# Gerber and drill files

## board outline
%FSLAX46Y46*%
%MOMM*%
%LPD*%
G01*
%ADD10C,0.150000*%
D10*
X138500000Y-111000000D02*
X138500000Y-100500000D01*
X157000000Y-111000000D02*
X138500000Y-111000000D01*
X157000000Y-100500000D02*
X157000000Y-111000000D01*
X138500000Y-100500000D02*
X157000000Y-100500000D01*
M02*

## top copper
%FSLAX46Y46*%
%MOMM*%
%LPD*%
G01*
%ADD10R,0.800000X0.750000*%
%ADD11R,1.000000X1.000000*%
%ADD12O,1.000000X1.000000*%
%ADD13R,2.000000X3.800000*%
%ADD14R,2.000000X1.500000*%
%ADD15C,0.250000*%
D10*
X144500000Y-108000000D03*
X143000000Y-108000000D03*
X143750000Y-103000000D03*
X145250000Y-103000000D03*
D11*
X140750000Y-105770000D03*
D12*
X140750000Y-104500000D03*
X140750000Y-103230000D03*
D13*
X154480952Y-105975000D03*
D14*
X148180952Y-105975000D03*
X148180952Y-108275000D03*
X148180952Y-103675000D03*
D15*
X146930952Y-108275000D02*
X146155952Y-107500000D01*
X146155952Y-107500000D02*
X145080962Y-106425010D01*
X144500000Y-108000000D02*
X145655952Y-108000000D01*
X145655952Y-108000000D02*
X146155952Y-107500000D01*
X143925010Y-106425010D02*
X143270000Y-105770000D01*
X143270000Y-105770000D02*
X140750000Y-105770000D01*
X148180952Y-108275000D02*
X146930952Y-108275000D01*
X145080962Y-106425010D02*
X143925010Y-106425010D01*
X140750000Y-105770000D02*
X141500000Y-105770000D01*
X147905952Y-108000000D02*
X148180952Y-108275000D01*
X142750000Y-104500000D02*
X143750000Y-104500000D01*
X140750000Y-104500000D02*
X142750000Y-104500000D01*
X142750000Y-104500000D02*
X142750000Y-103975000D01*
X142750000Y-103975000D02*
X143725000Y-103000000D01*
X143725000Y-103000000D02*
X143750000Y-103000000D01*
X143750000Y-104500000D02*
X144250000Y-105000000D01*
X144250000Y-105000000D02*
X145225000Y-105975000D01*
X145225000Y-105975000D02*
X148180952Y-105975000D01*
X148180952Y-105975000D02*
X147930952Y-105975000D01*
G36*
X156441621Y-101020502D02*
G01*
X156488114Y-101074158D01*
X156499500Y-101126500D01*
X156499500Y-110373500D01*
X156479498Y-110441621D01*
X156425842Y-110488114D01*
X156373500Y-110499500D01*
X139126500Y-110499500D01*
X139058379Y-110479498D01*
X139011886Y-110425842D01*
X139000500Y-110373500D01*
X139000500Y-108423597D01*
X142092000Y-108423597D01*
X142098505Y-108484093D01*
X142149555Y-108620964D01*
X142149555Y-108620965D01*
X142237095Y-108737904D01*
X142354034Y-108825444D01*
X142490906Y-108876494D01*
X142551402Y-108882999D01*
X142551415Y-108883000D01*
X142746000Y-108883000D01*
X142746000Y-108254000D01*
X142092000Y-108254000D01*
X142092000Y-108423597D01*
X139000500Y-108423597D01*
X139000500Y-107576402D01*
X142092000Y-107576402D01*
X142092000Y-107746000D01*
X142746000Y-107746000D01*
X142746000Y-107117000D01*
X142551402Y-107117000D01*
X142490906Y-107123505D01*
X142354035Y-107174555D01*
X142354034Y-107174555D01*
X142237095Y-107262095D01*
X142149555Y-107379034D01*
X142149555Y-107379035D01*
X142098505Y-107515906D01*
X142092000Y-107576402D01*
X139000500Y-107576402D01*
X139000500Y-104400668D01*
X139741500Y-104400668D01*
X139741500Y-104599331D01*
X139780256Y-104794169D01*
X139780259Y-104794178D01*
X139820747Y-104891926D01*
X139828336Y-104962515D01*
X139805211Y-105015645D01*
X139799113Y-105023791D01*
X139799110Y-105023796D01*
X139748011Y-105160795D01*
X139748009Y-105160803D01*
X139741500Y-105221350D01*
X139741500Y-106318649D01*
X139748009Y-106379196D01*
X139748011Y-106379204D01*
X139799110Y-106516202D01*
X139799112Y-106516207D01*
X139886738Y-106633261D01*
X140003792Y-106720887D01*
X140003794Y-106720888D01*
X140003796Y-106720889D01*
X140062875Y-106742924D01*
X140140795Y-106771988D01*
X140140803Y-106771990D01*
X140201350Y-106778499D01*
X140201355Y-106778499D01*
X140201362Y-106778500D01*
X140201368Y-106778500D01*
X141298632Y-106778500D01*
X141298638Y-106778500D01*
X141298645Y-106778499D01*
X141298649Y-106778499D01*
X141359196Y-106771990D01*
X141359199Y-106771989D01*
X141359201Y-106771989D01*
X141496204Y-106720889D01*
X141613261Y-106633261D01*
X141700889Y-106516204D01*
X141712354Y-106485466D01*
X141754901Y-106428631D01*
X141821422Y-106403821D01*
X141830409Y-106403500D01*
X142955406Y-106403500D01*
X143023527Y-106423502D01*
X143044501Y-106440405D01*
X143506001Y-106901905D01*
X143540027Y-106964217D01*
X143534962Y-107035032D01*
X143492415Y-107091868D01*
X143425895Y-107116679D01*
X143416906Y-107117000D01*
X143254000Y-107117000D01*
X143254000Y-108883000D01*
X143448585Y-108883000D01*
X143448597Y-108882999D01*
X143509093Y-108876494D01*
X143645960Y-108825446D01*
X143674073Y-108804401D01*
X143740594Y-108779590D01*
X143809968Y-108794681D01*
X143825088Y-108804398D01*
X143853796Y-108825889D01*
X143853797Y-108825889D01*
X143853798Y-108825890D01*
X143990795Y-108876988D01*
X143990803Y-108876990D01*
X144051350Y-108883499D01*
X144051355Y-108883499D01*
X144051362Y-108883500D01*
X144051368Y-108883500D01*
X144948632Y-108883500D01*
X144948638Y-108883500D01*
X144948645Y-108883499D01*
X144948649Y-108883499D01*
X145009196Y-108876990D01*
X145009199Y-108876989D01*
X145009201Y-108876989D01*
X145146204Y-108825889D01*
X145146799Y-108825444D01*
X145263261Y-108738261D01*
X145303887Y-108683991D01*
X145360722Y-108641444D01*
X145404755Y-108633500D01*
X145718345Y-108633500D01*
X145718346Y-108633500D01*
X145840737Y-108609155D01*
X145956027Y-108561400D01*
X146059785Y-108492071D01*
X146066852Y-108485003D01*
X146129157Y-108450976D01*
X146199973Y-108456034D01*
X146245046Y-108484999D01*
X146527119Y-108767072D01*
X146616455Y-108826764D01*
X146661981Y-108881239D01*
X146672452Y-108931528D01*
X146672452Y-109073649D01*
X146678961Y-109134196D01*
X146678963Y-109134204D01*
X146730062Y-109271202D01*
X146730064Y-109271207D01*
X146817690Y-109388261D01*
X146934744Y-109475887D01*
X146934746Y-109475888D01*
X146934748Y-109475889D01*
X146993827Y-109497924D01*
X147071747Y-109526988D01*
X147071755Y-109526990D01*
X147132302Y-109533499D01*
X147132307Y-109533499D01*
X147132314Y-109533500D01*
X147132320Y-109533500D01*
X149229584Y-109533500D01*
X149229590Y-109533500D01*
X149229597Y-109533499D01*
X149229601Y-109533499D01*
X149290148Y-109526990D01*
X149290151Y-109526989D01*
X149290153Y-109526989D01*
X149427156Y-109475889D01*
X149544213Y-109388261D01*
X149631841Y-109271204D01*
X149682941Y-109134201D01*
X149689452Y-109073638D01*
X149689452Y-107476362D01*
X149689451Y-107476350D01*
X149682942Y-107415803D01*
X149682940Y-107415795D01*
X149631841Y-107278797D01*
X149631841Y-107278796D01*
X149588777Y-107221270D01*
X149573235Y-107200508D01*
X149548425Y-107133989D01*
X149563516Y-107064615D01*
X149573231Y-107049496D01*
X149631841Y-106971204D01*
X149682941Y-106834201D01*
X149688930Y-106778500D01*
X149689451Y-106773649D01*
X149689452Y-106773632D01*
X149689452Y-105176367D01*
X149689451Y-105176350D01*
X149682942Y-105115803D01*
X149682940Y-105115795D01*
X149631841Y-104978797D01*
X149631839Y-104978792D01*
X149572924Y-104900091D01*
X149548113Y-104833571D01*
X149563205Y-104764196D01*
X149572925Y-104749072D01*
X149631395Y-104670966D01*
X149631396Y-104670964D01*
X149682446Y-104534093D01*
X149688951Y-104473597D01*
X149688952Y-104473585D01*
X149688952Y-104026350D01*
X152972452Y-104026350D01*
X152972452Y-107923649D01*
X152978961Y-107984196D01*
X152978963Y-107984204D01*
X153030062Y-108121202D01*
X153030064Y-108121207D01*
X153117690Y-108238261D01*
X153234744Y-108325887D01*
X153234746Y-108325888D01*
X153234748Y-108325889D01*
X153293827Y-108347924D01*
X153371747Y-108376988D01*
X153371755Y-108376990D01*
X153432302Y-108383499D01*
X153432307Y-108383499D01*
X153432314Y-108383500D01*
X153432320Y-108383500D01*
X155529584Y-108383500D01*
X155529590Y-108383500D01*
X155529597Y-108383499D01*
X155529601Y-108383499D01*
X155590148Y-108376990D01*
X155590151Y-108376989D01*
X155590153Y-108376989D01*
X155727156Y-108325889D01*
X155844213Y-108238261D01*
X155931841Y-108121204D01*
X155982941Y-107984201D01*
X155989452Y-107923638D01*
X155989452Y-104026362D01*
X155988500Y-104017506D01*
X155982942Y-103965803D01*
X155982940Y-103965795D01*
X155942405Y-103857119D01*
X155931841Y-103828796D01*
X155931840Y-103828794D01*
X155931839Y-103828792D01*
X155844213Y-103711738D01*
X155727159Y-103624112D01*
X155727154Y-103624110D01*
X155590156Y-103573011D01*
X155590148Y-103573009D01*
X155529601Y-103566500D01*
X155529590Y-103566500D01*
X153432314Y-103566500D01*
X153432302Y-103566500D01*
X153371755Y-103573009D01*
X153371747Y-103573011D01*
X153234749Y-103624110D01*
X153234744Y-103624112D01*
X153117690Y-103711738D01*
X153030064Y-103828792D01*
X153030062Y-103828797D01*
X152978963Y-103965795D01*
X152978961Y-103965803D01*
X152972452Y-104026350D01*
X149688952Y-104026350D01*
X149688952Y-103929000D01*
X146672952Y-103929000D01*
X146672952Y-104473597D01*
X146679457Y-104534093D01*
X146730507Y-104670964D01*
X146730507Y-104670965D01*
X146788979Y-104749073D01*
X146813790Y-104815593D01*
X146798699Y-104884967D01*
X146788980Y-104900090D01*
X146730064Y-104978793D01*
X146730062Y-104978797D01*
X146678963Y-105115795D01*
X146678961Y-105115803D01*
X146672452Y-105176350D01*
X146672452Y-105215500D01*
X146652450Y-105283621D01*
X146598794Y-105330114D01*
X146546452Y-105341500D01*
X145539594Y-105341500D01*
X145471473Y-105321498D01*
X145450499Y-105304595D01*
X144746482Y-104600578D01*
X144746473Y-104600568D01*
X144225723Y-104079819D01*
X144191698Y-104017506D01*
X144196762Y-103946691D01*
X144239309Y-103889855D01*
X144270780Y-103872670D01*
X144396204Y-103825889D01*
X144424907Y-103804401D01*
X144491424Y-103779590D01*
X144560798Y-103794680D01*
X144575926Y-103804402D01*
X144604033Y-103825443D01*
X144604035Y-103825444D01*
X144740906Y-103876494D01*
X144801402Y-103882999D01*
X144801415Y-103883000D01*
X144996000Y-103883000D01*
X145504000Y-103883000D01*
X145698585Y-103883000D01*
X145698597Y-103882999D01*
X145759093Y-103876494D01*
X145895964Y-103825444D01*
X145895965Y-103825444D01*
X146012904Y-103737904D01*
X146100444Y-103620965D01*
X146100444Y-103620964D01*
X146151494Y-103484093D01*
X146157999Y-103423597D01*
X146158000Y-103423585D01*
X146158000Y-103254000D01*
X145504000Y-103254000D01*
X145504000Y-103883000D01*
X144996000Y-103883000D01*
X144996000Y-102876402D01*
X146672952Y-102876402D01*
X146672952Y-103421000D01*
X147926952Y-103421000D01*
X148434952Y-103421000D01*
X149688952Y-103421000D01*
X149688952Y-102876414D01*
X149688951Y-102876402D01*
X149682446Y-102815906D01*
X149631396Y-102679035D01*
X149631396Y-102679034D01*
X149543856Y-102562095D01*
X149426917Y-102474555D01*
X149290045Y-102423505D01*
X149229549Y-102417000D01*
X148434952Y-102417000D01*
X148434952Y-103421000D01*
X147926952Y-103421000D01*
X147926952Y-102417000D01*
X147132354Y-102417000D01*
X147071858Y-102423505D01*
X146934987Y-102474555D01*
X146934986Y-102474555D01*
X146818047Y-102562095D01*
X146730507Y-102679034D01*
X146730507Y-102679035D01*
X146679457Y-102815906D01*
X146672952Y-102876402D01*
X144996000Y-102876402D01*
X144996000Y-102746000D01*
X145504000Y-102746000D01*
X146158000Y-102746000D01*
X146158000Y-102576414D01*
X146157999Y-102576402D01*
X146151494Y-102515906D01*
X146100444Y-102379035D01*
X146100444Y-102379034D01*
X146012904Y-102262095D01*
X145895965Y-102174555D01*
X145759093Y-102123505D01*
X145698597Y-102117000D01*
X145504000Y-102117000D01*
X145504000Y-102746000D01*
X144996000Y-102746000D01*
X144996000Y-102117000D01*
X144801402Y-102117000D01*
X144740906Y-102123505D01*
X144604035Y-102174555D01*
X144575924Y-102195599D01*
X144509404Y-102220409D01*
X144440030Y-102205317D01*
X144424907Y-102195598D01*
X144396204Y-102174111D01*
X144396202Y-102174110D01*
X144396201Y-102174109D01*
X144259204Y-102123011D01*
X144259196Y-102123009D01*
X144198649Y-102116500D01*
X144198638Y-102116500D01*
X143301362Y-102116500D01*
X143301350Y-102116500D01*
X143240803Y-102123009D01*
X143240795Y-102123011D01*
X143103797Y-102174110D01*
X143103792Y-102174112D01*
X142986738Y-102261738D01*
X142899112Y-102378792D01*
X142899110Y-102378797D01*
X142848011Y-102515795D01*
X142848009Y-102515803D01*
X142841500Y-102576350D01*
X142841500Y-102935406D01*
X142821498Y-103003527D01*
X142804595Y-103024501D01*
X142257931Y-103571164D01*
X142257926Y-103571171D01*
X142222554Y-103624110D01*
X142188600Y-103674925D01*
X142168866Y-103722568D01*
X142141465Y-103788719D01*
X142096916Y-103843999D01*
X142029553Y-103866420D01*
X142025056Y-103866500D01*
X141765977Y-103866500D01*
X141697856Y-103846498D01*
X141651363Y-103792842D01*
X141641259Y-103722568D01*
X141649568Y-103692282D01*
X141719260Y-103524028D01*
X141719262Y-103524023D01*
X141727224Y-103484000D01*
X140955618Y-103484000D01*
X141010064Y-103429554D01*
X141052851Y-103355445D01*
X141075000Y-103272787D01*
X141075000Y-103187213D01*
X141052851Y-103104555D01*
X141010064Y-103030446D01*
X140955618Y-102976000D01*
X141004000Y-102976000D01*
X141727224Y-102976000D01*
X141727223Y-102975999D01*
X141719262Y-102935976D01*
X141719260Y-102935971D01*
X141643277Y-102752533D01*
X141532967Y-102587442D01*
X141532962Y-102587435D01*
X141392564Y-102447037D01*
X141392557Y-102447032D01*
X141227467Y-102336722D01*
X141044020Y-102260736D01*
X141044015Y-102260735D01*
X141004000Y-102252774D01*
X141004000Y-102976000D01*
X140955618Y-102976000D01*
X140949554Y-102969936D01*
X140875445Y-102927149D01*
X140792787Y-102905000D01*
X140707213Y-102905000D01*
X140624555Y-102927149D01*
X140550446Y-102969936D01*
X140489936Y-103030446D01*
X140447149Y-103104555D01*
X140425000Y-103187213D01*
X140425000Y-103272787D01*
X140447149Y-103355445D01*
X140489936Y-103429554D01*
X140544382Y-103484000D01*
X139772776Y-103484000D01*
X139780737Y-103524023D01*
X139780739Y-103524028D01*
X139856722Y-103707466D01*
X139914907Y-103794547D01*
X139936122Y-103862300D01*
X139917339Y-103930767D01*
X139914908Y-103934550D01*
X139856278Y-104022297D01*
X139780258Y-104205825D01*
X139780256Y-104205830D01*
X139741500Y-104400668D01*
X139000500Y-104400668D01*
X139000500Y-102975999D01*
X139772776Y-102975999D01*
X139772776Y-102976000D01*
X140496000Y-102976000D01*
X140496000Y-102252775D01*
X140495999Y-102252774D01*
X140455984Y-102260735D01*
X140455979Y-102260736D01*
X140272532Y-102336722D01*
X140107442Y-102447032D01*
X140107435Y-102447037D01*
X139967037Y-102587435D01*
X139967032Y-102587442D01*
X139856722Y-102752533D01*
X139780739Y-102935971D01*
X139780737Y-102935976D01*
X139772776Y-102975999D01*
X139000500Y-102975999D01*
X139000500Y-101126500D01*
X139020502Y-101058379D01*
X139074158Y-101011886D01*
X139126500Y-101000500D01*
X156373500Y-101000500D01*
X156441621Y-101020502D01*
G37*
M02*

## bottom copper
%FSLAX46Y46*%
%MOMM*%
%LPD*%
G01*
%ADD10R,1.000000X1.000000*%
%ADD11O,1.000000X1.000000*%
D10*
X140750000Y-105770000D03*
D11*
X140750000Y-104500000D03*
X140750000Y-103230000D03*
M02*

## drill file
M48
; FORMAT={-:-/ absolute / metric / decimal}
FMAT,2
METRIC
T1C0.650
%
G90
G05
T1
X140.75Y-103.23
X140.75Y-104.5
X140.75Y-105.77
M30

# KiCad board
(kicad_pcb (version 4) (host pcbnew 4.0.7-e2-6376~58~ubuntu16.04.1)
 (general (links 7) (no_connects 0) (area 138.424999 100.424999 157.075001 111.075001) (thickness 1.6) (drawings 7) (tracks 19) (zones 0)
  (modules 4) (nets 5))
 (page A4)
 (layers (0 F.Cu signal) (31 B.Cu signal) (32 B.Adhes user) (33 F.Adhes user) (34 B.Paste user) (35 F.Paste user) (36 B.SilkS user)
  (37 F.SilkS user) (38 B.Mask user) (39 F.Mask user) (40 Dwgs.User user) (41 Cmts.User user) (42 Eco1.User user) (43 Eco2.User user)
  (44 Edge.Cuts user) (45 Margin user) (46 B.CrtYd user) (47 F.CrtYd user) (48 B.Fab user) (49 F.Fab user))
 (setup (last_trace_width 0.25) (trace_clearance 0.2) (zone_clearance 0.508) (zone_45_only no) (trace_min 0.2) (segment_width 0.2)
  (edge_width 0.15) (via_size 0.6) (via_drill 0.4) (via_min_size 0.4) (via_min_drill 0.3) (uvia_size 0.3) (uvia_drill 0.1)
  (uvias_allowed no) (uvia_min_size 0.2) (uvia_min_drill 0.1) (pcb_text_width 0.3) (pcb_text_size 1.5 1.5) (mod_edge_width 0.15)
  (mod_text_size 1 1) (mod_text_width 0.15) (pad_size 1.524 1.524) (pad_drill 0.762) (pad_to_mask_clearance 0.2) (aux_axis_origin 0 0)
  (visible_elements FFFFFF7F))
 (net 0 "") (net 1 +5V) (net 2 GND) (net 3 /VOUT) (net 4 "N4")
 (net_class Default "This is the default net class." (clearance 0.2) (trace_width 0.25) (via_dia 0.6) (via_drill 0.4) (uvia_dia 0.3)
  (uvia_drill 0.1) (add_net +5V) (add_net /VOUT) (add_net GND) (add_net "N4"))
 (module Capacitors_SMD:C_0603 (layer F.Cu) (at 143.75 108 180)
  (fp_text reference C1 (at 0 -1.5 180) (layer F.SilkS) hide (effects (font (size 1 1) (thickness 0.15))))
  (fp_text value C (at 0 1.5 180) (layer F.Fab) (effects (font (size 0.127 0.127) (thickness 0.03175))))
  (pad 1 smd rect (at -0.75 0 180) (size 0.8 0.75) (layers F.Cu F.Paste F.Mask) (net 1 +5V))
  (pad 2 smd rect (at 0.75 0 180) (size 0.8 0.75) (layers F.Cu F.Paste F.Mask) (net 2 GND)))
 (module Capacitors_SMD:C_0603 (layer F.Cu) (at 144.5 103)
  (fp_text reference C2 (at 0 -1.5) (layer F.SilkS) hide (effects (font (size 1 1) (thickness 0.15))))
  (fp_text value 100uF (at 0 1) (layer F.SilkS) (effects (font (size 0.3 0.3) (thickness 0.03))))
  (pad 1 smd rect (at -0.75 0) (size 0.8 0.75) (layers F.Cu F.Paste F.Mask) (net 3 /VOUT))
  (pad 2 smd rect (at 0.75 0) (size 0.8 0.75) (layers F.Cu F.Paste F.Mask) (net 2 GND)))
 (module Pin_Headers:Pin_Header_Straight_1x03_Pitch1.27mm (layer F.Cu) (at 140.75 105.77 180)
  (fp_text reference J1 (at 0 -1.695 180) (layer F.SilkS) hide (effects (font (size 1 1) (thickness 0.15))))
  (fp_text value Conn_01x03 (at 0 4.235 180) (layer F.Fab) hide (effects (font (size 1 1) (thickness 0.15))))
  (pad 1 thru_hole rect (at 0 0 180) (size 1 1) (drill 0.65) (layers *.Cu *.Mask) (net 1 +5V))
  (pad 2 thru_hole oval (at 0 1.27 180) (size 1 1) (drill 0.65) (layers *.Cu *.Mask) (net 3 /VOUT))
  (pad 3 thru_hole oval (at 0 2.54 180) (size 1 1) (drill 0.65) (layers *.Cu *.Mask) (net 2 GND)))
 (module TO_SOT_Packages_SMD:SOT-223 (layer F.Cu) (at 151.330952 105.975)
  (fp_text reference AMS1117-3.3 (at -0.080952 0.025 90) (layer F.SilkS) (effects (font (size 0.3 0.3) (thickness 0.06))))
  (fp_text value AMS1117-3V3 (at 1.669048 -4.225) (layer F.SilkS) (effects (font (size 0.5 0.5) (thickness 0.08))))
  (pad 4 smd rect (at 3.15 0) (size 2 3.8) (layers F.Cu F.Paste F.Mask) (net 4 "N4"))
  (pad 2 smd rect (at -3.15 0) (size 2 1.5) (layers F.Cu F.Paste F.Mask) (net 3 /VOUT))
  (pad 3 smd rect (at -3.15 2.3) (size 2 1.5) (layers F.Cu F.Paste F.Mask) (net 1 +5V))
  (pad 1 smd rect (at -3.15 -2.3) (size 2 1.5) (layers F.Cu F.Paste F.Mask) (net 2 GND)))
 (gr_line (start 138.5 111) (end 138.5 100.5) (angle 90) (layer Edge.Cuts) (width 0.15))
 (gr_line (start 157 111) (end 138.5 111) (angle 90) (layer Edge.Cuts) (width 0.15))
 (gr_line (start 157 100.5) (end 157 111) (angle 90) (layer Edge.Cuts) (width 0.15))
 (gr_line (start 138.5 100.5) (end 157 100.5) (angle 90) (layer Edge.Cuts) (width 0.15))
 (segment (start 146.930952 108.275) (end 146.155952 107.5) (width 0.25) (layer F.Cu) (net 1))
 (segment (start 146.155952 107.5) (end 145.080962 106.42501) (width 0.25) (layer F.Cu) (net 1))
 (segment (start 144.5 108) (end 145.655952 108) (width 0.25) (layer F.Cu) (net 1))
 (segment (start 145.655952 108) (end 146.155952 107.5) (width 0.25) (layer F.Cu) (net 1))
 (segment (start 143.92501 106.42501) (end 143.27 105.77) (width 0.25) (layer F.Cu) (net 1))
 (segment (start 143.27 105.77) (end 140.75 105.77) (width 0.25) (layer F.Cu) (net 1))
 (segment (start 148.180952 108.275) (end 146.930952 108.275) (width 0.25) (layer F.Cu) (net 1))
 (segment (start 145.080962 106.42501) (end 143.92501 106.42501) (width 0.25) (layer F.Cu) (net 1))
 (segment (start 140.75 105.77) (end 141.5 105.77) (width 0.25) (layer F.Cu) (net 1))
 (segment (start 147.905952 108) (end 148.180952 108.275) (width 0.25) (layer F.Cu) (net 1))
 (segment (start 142.75 104.5) (end 143.75 104.5) (width 0.25) (layer F.Cu) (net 3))
 (segment (start 140.75 104.5) (end 142.75 104.5) (width 0.25) (layer F.Cu) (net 3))
 (segment (start 142.75 104.5) (end 142.75 103.975) (width 0.25) (layer F.Cu) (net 3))
 (segment (start 142.75 103.975) (end 143.725 103) (width 0.25) (layer F.Cu) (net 3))
 (segment (start 143.725 103) (end 143.75 103) (width 0.25) (layer F.Cu) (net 3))
 (segment (start 143.75 104.5) (end 144.25 105) (width 0.25) (layer F.Cu) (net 3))
 (segment (start 144.25 105) (end 145.225 105.975) (width 0.25) (layer F.Cu) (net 3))
 (segment (start 145.225 105.975) (end 148.180952 105.975) (width 0.25) (layer F.Cu) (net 3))
 (segment (start 148.180952 105.975) (end 147.930952 105.975) (width 0.25) (layer F.Cu) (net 3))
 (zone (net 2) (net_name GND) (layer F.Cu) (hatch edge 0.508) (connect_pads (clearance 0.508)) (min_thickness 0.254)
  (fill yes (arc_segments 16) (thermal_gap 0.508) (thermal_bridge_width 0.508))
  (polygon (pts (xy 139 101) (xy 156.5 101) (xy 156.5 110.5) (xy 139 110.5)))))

